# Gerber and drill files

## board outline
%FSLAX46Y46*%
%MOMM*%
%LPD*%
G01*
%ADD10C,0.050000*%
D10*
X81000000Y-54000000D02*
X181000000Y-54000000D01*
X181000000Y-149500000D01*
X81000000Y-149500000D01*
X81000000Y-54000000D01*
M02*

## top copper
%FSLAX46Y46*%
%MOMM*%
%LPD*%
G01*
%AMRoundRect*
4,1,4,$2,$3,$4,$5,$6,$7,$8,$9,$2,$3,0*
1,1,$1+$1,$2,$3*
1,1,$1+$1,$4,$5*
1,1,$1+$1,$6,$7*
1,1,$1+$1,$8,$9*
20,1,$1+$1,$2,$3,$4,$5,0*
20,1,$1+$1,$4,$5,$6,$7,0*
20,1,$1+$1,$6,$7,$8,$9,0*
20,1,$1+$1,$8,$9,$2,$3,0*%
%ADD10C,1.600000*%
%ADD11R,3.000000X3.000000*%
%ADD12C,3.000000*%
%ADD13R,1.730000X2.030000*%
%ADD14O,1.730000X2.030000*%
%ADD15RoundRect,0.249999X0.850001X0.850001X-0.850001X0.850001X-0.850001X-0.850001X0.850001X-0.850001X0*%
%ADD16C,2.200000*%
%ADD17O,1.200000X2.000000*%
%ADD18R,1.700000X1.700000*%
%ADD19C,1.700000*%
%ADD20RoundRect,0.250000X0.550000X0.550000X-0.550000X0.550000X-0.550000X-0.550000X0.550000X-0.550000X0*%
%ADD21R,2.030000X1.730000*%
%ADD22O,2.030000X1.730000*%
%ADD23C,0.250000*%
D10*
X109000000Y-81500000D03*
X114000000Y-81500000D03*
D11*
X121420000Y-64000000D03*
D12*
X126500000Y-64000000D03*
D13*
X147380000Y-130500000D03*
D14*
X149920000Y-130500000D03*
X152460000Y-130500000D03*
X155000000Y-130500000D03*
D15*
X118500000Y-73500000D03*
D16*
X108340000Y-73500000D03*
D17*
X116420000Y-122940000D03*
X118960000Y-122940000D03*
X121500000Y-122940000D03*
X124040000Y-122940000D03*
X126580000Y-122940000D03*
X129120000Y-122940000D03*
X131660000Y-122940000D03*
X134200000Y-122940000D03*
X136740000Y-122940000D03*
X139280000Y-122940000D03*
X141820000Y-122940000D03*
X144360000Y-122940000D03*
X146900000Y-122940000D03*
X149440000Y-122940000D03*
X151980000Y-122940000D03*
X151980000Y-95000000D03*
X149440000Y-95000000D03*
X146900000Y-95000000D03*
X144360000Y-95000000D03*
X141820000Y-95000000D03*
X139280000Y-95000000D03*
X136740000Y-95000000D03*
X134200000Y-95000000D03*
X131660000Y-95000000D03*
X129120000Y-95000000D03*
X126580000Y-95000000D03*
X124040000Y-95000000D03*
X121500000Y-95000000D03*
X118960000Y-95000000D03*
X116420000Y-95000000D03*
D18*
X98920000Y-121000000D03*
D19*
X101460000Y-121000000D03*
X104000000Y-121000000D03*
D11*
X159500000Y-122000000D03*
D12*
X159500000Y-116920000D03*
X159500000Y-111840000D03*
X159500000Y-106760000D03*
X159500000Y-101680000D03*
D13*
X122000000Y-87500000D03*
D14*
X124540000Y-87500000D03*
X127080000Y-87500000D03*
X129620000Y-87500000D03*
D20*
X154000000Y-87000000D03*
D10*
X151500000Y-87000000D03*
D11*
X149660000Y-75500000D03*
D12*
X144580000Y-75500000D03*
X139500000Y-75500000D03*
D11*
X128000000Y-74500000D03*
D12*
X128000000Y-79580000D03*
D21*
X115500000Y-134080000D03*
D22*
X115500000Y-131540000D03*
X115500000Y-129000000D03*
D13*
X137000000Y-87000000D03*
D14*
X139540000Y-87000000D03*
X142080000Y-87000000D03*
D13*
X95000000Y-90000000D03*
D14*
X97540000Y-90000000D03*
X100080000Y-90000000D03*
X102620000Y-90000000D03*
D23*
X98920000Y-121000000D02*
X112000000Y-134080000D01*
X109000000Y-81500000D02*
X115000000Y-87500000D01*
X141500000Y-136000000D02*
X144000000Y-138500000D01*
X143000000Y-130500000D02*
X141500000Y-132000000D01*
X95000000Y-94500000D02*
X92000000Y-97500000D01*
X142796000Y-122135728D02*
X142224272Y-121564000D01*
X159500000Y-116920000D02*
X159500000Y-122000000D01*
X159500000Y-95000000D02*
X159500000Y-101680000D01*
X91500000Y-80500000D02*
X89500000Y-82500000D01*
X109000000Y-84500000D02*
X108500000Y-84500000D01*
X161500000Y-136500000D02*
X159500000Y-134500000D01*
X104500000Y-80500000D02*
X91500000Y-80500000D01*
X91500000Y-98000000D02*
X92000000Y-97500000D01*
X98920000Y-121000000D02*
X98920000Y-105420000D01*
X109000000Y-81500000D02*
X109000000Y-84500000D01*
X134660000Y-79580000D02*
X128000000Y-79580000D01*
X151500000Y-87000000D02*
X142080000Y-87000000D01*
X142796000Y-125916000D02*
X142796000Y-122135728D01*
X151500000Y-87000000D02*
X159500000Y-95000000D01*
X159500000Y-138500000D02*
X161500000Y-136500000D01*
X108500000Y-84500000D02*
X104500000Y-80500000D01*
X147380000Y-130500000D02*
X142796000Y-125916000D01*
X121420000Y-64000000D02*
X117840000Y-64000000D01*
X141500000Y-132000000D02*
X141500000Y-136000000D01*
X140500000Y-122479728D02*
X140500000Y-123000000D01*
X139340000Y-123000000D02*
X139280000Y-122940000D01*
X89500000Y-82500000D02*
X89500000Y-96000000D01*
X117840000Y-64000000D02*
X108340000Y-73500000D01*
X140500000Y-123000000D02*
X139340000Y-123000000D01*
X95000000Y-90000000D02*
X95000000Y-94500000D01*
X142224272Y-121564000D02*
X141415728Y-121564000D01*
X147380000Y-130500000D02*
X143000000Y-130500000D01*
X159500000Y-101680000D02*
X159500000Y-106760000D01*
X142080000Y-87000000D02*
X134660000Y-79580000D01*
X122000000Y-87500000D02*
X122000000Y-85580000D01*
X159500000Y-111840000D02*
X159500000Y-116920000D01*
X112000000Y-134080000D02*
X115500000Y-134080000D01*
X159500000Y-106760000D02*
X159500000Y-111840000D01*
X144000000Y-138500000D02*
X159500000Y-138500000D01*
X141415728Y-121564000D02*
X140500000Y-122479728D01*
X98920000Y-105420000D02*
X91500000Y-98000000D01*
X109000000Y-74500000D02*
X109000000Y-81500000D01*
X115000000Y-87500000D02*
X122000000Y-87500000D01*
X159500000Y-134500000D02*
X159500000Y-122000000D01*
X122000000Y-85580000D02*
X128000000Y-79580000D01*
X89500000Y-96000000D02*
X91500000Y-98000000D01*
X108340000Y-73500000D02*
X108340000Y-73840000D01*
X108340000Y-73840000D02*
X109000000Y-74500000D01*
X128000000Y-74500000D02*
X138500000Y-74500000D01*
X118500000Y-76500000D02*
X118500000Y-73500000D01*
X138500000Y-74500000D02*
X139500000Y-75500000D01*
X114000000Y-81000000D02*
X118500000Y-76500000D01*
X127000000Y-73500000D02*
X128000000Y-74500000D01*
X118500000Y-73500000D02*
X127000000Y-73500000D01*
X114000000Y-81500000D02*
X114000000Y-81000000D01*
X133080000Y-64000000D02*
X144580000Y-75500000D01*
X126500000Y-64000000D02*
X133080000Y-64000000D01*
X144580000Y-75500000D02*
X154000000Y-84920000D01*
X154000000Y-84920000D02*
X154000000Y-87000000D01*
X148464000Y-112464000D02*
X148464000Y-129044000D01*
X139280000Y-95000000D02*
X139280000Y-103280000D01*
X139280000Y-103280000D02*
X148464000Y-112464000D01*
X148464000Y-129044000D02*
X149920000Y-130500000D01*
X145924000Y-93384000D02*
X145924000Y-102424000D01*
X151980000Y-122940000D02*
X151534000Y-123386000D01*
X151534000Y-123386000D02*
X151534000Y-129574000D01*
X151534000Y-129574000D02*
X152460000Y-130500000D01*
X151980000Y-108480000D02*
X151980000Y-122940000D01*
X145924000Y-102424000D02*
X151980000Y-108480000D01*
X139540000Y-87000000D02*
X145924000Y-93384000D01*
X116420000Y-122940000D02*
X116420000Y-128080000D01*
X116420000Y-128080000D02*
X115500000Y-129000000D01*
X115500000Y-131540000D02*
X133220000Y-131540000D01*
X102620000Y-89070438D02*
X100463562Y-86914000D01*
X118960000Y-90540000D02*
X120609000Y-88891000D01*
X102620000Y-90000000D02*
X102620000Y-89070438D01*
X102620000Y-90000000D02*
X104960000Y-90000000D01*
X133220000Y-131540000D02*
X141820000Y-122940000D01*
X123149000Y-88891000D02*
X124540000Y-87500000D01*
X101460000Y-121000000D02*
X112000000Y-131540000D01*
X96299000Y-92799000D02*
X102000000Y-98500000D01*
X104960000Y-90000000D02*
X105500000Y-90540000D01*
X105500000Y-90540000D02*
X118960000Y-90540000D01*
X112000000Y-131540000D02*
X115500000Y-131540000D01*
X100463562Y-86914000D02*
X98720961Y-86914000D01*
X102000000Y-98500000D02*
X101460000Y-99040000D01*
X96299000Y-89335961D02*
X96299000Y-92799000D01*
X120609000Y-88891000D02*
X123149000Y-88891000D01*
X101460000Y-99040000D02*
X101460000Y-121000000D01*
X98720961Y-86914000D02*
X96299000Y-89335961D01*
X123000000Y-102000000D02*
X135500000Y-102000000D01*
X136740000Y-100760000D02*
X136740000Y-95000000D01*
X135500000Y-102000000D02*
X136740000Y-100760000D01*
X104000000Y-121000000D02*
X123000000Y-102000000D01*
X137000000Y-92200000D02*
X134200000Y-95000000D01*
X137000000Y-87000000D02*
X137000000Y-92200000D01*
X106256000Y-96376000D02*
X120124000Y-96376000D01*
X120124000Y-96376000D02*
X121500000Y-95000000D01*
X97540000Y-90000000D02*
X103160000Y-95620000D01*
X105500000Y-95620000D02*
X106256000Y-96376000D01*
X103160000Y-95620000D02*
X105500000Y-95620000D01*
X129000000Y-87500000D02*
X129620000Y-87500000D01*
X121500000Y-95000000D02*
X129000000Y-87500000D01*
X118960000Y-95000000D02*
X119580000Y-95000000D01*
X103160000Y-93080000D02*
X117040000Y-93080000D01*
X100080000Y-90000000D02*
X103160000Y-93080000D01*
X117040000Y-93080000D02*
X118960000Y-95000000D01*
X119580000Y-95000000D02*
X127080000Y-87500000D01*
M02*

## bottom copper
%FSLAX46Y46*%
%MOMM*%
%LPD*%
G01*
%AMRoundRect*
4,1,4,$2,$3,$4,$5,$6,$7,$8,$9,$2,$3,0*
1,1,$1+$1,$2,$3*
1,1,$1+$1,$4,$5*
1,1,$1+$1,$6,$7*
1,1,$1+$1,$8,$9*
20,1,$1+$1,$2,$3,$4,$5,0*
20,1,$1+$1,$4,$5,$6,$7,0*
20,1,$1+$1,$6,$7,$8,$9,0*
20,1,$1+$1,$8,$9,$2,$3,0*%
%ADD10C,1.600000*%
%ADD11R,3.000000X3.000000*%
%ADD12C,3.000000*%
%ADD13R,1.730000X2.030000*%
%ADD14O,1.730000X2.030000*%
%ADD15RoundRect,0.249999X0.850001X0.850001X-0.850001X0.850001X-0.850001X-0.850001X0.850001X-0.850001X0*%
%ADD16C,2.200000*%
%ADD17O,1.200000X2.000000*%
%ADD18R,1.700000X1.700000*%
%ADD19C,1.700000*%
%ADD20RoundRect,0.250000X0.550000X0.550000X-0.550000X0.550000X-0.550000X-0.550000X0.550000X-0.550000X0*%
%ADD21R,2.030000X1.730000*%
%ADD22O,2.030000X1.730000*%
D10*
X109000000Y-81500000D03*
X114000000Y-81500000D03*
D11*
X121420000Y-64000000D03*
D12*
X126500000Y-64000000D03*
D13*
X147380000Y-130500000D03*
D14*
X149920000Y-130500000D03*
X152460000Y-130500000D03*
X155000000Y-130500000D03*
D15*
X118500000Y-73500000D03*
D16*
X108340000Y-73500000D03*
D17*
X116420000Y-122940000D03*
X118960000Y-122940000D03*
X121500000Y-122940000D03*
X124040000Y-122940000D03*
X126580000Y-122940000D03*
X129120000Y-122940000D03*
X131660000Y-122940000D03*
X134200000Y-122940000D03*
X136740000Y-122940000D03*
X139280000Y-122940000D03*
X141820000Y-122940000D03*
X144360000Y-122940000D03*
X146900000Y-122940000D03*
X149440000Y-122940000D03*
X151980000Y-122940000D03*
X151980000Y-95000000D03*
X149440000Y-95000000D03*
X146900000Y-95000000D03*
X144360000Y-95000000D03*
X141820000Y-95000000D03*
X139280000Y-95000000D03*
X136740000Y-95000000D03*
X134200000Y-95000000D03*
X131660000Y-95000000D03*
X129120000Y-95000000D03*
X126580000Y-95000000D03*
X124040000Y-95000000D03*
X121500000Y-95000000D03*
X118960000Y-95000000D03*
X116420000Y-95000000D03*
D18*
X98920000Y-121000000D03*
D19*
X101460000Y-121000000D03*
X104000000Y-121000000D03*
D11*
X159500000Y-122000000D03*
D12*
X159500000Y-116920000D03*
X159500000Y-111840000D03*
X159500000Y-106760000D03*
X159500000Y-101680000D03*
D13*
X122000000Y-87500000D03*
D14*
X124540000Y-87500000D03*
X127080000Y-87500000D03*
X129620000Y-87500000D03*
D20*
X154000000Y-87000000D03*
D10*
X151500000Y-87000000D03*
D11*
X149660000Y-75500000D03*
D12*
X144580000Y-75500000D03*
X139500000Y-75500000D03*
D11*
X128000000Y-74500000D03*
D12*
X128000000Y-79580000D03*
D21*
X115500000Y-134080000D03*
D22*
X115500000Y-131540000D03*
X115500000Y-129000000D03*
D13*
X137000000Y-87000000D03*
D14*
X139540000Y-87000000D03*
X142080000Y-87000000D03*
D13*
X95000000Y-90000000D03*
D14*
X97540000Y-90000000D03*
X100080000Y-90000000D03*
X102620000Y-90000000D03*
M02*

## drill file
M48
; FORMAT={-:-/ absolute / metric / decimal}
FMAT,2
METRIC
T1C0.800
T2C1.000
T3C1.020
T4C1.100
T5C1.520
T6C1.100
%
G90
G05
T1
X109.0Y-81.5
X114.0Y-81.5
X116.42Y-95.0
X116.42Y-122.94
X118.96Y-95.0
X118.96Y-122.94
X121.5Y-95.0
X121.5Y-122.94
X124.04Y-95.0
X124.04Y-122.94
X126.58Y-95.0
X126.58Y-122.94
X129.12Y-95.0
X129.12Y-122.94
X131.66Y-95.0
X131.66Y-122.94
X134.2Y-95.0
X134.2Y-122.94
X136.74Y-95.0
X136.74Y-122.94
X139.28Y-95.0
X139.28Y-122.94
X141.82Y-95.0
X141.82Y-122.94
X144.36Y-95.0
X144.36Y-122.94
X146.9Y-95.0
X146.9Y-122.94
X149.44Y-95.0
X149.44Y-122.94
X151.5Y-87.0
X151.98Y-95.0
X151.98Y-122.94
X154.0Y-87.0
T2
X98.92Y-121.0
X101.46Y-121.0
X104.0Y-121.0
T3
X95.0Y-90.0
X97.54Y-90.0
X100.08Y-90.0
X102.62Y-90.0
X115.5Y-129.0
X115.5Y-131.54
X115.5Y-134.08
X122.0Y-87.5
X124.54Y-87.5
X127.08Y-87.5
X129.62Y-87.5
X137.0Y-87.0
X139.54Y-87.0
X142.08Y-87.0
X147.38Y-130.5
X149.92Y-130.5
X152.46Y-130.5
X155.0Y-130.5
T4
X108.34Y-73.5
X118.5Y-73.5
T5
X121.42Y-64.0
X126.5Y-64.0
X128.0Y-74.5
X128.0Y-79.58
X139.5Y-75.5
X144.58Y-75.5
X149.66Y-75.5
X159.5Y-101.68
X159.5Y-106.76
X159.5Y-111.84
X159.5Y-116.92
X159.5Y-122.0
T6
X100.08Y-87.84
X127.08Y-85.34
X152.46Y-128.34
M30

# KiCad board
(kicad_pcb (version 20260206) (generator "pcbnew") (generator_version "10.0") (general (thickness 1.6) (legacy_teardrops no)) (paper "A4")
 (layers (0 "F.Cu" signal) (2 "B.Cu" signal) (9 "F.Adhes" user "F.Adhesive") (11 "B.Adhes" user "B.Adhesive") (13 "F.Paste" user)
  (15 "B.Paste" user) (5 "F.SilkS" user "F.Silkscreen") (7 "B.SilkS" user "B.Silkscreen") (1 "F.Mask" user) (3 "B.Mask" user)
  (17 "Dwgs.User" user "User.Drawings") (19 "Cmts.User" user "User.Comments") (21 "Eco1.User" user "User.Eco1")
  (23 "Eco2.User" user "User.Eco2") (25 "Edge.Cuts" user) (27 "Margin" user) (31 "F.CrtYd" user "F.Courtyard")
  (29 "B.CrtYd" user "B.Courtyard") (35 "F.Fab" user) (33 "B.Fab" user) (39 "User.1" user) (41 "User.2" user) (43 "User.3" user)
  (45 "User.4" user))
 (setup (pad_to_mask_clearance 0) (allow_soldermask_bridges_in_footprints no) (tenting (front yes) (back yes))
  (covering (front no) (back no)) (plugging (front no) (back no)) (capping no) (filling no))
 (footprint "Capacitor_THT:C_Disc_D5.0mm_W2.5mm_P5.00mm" (layer "F.Cu") (at 109 81.5)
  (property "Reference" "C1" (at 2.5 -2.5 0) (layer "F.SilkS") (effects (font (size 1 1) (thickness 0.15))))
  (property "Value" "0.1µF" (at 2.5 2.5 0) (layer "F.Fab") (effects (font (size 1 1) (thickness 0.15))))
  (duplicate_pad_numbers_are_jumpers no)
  (pad "1" thru_hole circle (at 0 0) (size 1.6 1.6) (drill 0.8) (layers "*.Cu" "*.Mask") (remove_unused_layers no) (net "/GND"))
  (pad "2" thru_hole circle (at 5 0) (size 1.6 1.6) (drill 0.8) (layers "*.Cu" "*.Mask") (remove_unused_layers no) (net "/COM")))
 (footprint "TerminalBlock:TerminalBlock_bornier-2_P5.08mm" (layer "F.Cu") (at 121.42 64)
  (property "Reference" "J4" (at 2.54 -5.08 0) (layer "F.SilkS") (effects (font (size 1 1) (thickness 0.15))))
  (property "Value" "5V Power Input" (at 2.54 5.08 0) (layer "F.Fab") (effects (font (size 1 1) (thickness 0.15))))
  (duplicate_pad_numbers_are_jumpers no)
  (pad "1" thru_hole rect (at 0 0) (size 3 3) (drill 1.52) (layers "*.Cu" "*.Mask") (remove_unused_layers no) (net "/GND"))
  (pad "2" thru_hole circle (at 5.08 0) (size 3 3) (drill 1.52) (layers "*.Cu" "*.Mask") (remove_unused_layers no) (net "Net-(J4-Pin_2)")))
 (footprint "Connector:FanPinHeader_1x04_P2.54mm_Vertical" (layer "F.Cu") (at 147.38 130.5)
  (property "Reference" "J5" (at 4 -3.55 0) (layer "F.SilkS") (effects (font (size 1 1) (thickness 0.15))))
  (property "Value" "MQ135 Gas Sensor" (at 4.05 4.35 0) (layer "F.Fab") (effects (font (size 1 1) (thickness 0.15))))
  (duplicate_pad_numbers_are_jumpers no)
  (pad "" np_thru_hole circle (at 5.08 -2.16 90) (size 1.1 1.1) (drill 1.1) (layers "*.Cu" "*.Mask"))
  (pad "1" thru_hole rect (at 0 0 90) (size 2.03 1.73) (drill 1.02) (layers "*.Cu" "*.Mask") (remove_unused_layers no) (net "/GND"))
  (pad "2" thru_hole oval (at 2.54 0 90) (size 2.03 1.73) (drill 1.02) (layers "*.Cu" "*.Mask") (remove_unused_layers no)
   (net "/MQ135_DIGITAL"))
  (pad "3" thru_hole oval (at 5.08 0 90) (size 2.03 1.73) (drill 1.02) (layers "*.Cu" "*.Mask") (remove_unused_layers no) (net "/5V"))
  (pad "4" thru_hole oval (at 7.62 0 90) (size 2.03 1.73) (drill 1.02) (layers "*.Cu" "*.Mask") (remove_unused_layers no) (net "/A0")))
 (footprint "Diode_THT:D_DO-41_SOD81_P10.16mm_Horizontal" (layer "F.Cu") (at 118.5 73.5 180)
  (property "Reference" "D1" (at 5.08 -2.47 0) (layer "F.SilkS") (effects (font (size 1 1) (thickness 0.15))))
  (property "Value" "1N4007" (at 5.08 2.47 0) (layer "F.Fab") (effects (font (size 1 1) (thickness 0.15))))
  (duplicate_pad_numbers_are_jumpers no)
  (pad "1" thru_hole roundrect (at 0 0 180) (size 2.2 2.2) (drill 1.1) (layers "*.Cu" "*.Mask") (remove_unused_layers no)
   (roundrect_rratio 0.113636) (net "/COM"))
  (pad "2" thru_hole circle (at 10.16 0 180) (size 2.2 2.2) (drill 1.1) (layers "*.Cu" "*.Mask") (remove_unused_layers no) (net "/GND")))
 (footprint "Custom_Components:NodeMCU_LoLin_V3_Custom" (layer "F.Cu") (at 134.2 108.97)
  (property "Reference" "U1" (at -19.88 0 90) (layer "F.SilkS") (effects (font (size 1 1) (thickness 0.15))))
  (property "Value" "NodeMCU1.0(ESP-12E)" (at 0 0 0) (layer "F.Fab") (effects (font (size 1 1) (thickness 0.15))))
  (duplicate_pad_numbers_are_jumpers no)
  (pad "1" thru_hole oval (at -17.78 13.97) (size 1.2 2) (drill 0.8) (layers "*.Cu" "*.Mask") (remove_unused_layers no)
   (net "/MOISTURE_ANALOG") (thermal_bridge_angle 45))
  (pad "2" thru_hole oval (at -15.24 13.97) (size 1.2 2) (drill 0.8) (layers "*.Cu" "*.Mask") (remove_unused_layers no)
   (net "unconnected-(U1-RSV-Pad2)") (thermal_bridge_angle 45))
  (pad "3" thru_hole oval (at -12.7 13.97) (size 1.2 2) (drill 0.8) (layers "*.Cu" "*.Mask") (remove_unused_layers no)
   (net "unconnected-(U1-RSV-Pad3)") (thermal_bridge_angle 45))
  (pad "4" thru_hole oval (at -10.16 13.97) (size 1.2 2) (drill 0.8) (layers "*.Cu" "*.Mask") (remove_unused_layers no)
   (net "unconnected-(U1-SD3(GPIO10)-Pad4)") (thermal_bridge_angle 45))
  (pad "5" thru_hole oval (at -7.62 13.97) (size 1.2 2) (drill 0.8) (layers "*.Cu" "*.Mask") (remove_unused_layers no)
   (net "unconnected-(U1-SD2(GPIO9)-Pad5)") (thermal_bridge_angle 45))
  (pad "6" thru_hole oval (at -5.08 13.97) (size 1.2 2) (drill 0.8) (layers "*.Cu" "*.Mask") (remove_unused_layers no)
   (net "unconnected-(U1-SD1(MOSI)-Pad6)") (thermal_bridge_angle 45))
  (pad "7" thru_hole oval (at -2.54 13.97) (size 1.2 2) (drill 0.8) (layers "*.Cu" "*.Mask") (remove_unused_layers no)
   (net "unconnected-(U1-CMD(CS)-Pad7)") (thermal_bridge_angle 45))
  (pad "8" thru_hole oval (at 0 13.97) (size 1.2 2) (drill 0.8) (layers "*.Cu" "*.Mask") (remove_unused_layers no)
   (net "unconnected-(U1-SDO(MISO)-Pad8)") (thermal_bridge_angle 45))
  (pad "9" thru_hole oval (at 2.54 13.97) (size 1.2 2) (drill 0.8) (layers "*.Cu" "*.Mask") (remove_unused_layers no)
   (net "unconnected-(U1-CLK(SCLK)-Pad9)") (thermal_bridge_angle 45))
  (pad "10" thru_hole oval (at 5.08 13.97) (size 1.2 2) (drill 0.8) (layers "*.Cu" "*.Mask") (remove_unused_layers no) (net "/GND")
   (thermal_bridge_angle 45))
  (pad "11" thru_hole oval (at 7.62 13.97) (size 1.2 2) (drill 0.8) (layers "*.Cu" "*.Mask") (remove_unused_layers no) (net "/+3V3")
   (thermal_bridge_angle 45))
  (pad "12" thru_hole oval (at 10.16 13.97) (size 1.2 2) (drill 0.8) (layers "*.Cu" "*.Mask") (remove_unused_layers no)
   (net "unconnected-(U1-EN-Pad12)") (thermal_bridge_angle 45))
  (pad "13" thru_hole oval (at 12.7 13.97) (size 1.2 2) (drill 0.8) (layers "*.Cu" "*.Mask") (remove_unused_layers no)
   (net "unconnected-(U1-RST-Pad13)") (thermal_bridge_angle 45))
  (pad "14" thru_hole oval (at 15.24 13.97) (size 1.2 2) (drill 0.8) (layers "*.Cu" "*.Mask") (remove_unused_layers no)
   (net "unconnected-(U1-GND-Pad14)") (thermal_bridge_angle 45))
  (pad "15" thru_hole oval (at 17.78 13.97) (size 1.2 2) (drill 0.8) (layers "*.Cu" "*.Mask") (remove_unused_layers no) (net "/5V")
   (thermal_bridge_angle 45))
  (pad "16" thru_hole oval (at 17.78 -13.97) (size 1.2 2) (drill 0.8) (layers "*.Cu" "*.Mask") (remove_unused_layers no)
   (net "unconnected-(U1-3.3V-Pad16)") (thermal_bridge_angle 45))
  (pad "17" thru_hole oval (at 15.24 -13.97) (size 1.2 2) (drill 0.8) (layers "*.Cu" "*.Mask") (remove_unused_layers no)
   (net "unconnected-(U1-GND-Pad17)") (thermal_bridge_angle 45))
  (pad "18" thru_hole oval (at 12.7 -13.97) (size 1.2 2) (drill 0.8) (layers "*.Cu" "*.Mask") (remove_unused_layers no)
   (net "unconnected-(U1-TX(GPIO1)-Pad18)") (thermal_bridge_angle 45))
  (pad "19" thru_hole oval (at 10.16 -13.97) (size 1.2 2) (drill 0.8) (layers "*.Cu" "*.Mask") (remove_unused_layers no)
   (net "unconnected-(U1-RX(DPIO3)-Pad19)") (thermal_bridge_angle 45))
  (pad "20" thru_hole oval (at 7.62 -13.97) (size 1.2 2) (drill 0.8) (layers "*.Cu" "*.Mask") (remove_unused_layers no)
   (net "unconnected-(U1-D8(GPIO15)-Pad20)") (thermal_bridge_angle 45))
  (pad "21" thru_hole oval (at 5.08 -13.97) (size 1.2 2) (drill 0.8) (layers "*.Cu" "*.Mask") (remove_unused_layers no)
   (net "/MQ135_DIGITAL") (thermal_bridge_angle 45))
  (pad "22" thru_hole oval (at 2.54 -13.97) (size 1.2 2) (drill 0.8) (layers "*.Cu" "*.Mask") (remove_unused_layers no) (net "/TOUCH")
   (thermal_bridge_angle 45))
  (pad "23" thru_hole oval (at 0 -13.97) (size 1.2 2) (drill 0.8) (layers "*.Cu" "*.Mask") (remove_unused_layers no) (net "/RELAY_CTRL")
   (thermal_bridge_angle 45))
  (pad "24" thru_hole oval (at -2.54 -13.97) (size 1.2 2) (drill 0.8) (layers "*.Cu" "*.Mask") (remove_unused_layers no)
   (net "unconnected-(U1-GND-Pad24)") (thermal_bridge_angle 45))
  (pad "25" thru_hole oval (at -5.08 -13.97) (size 1.2 2) (drill 0.8) (layers "*.Cu" "*.Mask") (remove_unused_layers no)
   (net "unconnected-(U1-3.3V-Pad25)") (thermal_bridge_angle 45))
  (pad "26" thru_hole oval (at -7.62 -13.97) (size 1.2 2) (drill 0.8) (layers "*.Cu" "*.Mask") (remove_unused_layers no)
   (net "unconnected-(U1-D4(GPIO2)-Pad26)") (thermal_bridge_angle 45))
  (pad "27" thru_hole oval (at -10.16 -13.97) (size 1.2 2) (drill 0.8) (layers "*.Cu" "*.Mask") (remove_unused_layers no)
   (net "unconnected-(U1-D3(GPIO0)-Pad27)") (thermal_bridge_angle 45))
  (pad "28" thru_hole oval (at -12.7 -13.97) (size 1.2 2) (drill 0.8) (layers "*.Cu" "*.Mask") (remove_unused_layers no) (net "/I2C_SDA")
   (thermal_bridge_angle 45))
  (pad "29" thru_hole oval (at -15.24 -13.97) (size 1.2 2) (drill 0.8) (layers "*.Cu" "*.Mask") (remove_unused_layers no) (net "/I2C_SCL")
   (thermal_bridge_angle 45))
  (pad "30" thru_hole oval (at -17.78 -13.97) (size 1.2 2) (drill 0.8) (layers "*.Cu" "*.Mask") (remove_unused_layers no)
   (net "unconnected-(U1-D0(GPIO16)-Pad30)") (thermal_bridge_angle 45)))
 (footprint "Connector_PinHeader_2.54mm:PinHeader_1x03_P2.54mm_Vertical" (layer "F.Cu") (at 98.92 121 90)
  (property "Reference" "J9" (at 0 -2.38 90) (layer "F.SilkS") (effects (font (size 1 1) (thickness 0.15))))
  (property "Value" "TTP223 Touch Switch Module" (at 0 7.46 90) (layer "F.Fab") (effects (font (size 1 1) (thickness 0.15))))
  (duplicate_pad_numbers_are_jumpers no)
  (pad "1" thru_hole rect (at 0 0 90) (size 1.7 1.7) (drill 1) (layers "*.Cu" "*.Mask") (remove_unused_layers no) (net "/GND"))
  (pad "2" thru_hole circle (at 0 2.54 90) (size 1.7 1.7) (drill 1) (layers "*.Cu" "*.Mask") (remove_unused_layers no) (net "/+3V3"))
  (pad "3" thru_hole circle (at 0 5.08 90) (size 1.7 1.7) (drill 1) (layers "*.Cu" "*.Mask") (remove_unused_layers no) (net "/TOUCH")))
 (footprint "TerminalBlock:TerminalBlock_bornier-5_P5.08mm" (layer "F.Cu") (at 159.5 122 90)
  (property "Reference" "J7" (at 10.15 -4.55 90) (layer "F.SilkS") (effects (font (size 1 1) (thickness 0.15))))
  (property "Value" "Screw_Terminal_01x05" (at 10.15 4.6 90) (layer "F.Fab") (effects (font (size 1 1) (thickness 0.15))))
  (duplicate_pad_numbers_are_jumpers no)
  (pad "1" thru_hole rect (at 0 0 90) (size 3 3) (drill 1.52) (layers "*.Cu" "*.Mask") (remove_unused_layers no) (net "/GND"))
  (pad "2" thru_hole circle (at 5.08 0 90) (size 3 3) (drill 1.52) (layers "*.Cu" "*.Mask") (remove_unused_layers no) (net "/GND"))
  (pad "3" thru_hole circle (at 10.16 0 90) (size 3 3) (drill 1.52) (layers "*.Cu" "*.Mask") (remove_unused_layers no) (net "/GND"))
  (pad "4" thru_hole circle (at 15.24 0 90) (size 3 3) (drill 1.52) (layers "*.Cu" "*.Mask") (remove_unused_layers no) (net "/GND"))
  (pad "5" thru_hole circle (at 20.32 0 90) (size 3 3) (drill 1.52) (layers "*.Cu" "*.Mask") (remove_unused_layers no) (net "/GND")))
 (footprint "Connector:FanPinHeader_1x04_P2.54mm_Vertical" (layer "F.Cu") (at 122 87.5)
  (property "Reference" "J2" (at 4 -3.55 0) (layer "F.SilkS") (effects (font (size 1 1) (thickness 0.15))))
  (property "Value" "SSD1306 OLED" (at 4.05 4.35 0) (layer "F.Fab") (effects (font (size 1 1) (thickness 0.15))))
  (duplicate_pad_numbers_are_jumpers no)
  (pad "" np_thru_hole circle (at 5.08 -2.16 90) (size 1.1 1.1) (drill 1.1) (layers "*.Cu" "*.Mask"))
  (pad "1" thru_hole rect (at 0 0 90) (size 2.03 1.73) (drill 1.02) (layers "*.Cu" "*.Mask") (remove_unused_layers no) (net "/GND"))
  (pad "2" thru_hole oval (at 2.54 0 90) (size 2.03 1.73) (drill 1.02) (layers "*.Cu" "*.Mask") (remove_unused_layers no) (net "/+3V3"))
  (pad "3" thru_hole oval (at 5.08 0 90) (size 2.03 1.73) (drill 1.02) (layers "*.Cu" "*.Mask") (remove_unused_layers no) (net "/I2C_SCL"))
  (pad "4" thru_hole oval (at 7.62 0 90) (size 2.03 1.73) (drill 1.02) (layers "*.Cu" "*.Mask") (remove_unused_layers no) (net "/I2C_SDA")))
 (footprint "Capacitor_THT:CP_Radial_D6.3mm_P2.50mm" (layer "F.Cu") (at 154 87 180)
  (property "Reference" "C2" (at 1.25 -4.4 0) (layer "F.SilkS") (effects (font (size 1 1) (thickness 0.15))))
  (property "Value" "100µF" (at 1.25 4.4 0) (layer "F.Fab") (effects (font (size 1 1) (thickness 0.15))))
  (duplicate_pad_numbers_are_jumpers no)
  (pad "1" thru_hole roundrect (at 0 0 180) (size 1.6 1.6) (drill 0.8) (layers "*.Cu" "*.Mask") (remove_unused_layers no)
   (roundrect_rratio 0.15625) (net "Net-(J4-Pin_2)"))
  (pad "2" thru_hole circle (at 2.5 0 180) (size 1.6 1.6) (drill 0.8) (layers "*.Cu" "*.Mask") (remove_unused_layers no) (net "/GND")))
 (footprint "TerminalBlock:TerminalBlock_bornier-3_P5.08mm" (layer "F.Cu") (at 149.66 75.5 180)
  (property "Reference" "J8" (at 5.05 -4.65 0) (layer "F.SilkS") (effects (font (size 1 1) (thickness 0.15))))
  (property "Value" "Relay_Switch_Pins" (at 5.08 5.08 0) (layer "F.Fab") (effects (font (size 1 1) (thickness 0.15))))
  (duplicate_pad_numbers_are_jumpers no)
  (pad "1" thru_hole rect (at 0 0 180) (size 3 3) (drill 1.52) (layers "*.Cu" "*.Mask") (remove_unused_layers no)
   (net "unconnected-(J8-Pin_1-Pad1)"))
  (pad "2" thru_hole circle (at 5.08 0 180) (size 3 3) (drill 1.52) (layers "*.Cu" "*.Mask") (remove_unused_layers no)
   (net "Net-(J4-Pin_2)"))
  (pad "3" thru_hole circle (at 10.16 0 180) (size 3 3) (drill 1.52) (layers "*.Cu" "*.Mask") (remove_unused_layers no) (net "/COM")))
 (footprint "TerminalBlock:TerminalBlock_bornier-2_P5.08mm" (layer "F.Cu") (at 128 74.5 -90)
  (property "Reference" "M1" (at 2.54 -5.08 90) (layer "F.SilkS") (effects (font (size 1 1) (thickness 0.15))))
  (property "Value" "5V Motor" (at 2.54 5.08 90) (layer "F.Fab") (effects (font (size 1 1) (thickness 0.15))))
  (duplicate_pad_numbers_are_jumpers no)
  (pad "1" thru_hole rect (at 0 0 270) (size 3 3) (drill 1.52) (layers "*.Cu" "*.Mask") (remove_unused_layers no) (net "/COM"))
  (pad "2" thru_hole circle (at 5.08 0 270) (size 3 3) (drill 1.52) (layers "*.Cu" "*.Mask") (remove_unused_layers no) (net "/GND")))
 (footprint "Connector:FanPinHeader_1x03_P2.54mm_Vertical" (layer "F.Cu") (at 115.5 134.08 90)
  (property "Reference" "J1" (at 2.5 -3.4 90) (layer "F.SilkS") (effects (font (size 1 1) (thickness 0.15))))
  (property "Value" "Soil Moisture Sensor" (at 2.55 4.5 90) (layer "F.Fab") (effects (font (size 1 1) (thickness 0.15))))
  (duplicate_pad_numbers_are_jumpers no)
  (pad "1" thru_hole rect (at 0 0 180) (size 2.03 1.73) (drill 1.02) (layers "*.Cu" "*.Mask") (remove_unused_layers no) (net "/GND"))
  (pad "2" thru_hole oval (at 2.54 0 180) (size 2.03 1.73) (drill 1.02) (layers "*.Cu" "*.Mask") (remove_unused_layers no) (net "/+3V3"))
  (pad "3" thru_hole oval (at 5.08 0 180) (size 2.03 1.73) (drill 1.02) (layers "*.Cu" "*.Mask") (remove_unused_layers no)
   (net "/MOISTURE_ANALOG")))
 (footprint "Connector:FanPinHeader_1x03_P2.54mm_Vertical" (layer "F.Cu") (at 137 87)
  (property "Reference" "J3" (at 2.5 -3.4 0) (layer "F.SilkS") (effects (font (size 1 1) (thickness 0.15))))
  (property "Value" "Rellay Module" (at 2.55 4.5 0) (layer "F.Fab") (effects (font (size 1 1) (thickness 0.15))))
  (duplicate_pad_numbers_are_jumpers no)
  (pad "1" thru_hole rect (at 0 0 90) (size 2.03 1.73) (drill 1.02) (layers "*.Cu" "*.Mask") (remove_unused_layers no) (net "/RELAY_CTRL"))
  (pad "2" thru_hole oval (at 2.54 0 90) (size 2.03 1.73) (drill 1.02) (layers "*.Cu" "*.Mask") (remove_unused_layers no) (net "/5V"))
  (pad "3" thru_hole oval (at 5.08 0 90) (size 2.03 1.73) (drill 1.02) (layers "*.Cu" "*.Mask") (remove_unused_layers no) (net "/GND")))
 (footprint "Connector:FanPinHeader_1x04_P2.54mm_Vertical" (layer "F.Cu") (at 95 90)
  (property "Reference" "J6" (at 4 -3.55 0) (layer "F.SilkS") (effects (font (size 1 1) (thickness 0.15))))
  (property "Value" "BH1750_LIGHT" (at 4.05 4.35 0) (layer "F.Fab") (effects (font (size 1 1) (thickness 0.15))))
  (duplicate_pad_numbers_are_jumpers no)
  (pad "" np_thru_hole circle (at 5.08 -2.16 90) (size 1.1 1.1) (drill 1.1) (layers "*.Cu" "*.Mask"))
  (pad "1" thru_hole rect (at 0 0 90) (size 2.03 1.73) (drill 1.02) (layers "*.Cu" "*.Mask") (remove_unused_layers no) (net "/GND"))
  (pad "2" thru_hole oval (at 2.54 0 90) (size 2.03 1.73) (drill 1.02) (layers "*.Cu" "*.Mask") (remove_unused_layers no) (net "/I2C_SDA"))
  (pad "3" thru_hole oval (at 5.08 0 90) (size 2.03 1.73) (drill 1.02) (layers "*.Cu" "*.Mask") (remove_unused_layers no) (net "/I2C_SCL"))
  (pad "4" thru_hole oval (at 7.62 0 90) (size 2.03 1.73) (drill 1.02) (layers "*.Cu" "*.Mask") (remove_unused_layers no) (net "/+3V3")))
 (gr_rect (start 81 54) (end 181 149.5) (stroke (width 0.05) (type default)) (fill no) (layer "Edge.Cuts"))
 (segment (start 98.92 121) (end 112 134.08) (width 0.25) (layer "F.Cu") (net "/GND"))
 (segment (start 109 81.5) (end 115 87.5) (width 0.25) (layer "F.Cu") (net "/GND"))
 (segment (start 141.5 136) (end 144 138.5) (width 0.25) (layer "F.Cu") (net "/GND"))
 (segment (start 143 130.5) (end 141.5 132) (width 0.25) (layer "F.Cu") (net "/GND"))
 (segment (start 95 94.5) (end 92 97.5) (width 0.25) (layer "F.Cu") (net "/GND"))
 (segment (start 142.796 122.135728) (end 142.224272 121.564) (width 0.25) (layer "F.Cu") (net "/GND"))
 (segment (start 159.5 116.92) (end 159.5 122) (width 0.25) (layer "F.Cu") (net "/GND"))
 (segment (start 159.5 95) (end 159.5 101.68) (width 0.25) (layer "F.Cu") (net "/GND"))
 (segment (start 91.5 80.5) (end 89.5 82.5) (width 0.25) (layer "F.Cu") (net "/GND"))
 (segment (start 109 84.5) (end 108.5 84.5) (width 0.25) (layer "F.Cu") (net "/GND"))
 (segment (start 161.5 136.5) (end 159.5 134.5) (width 0.25) (layer "F.Cu") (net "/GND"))
 (segment (start 104.5 80.5) (end 91.5 80.5) (width 0.25) (layer "F.Cu") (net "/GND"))
 (segment (start 91.5 98) (end 92 97.5) (width 0.25) (layer "F.Cu") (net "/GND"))
 (segment (start 98.92 121) (end 98.92 105.42) (width 0.25) (layer "F.Cu") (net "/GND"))
 (segment (start 109 81.5) (end 109 84.5) (width 0.25) (layer "F.Cu") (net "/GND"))
 (segment (start 134.66 79.58) (end 128 79.58) (width 0.25) (layer "F.Cu") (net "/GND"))
 (segment (start 151.5 87) (end 142.08 87) (width 0.25) (layer "F.Cu") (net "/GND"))
 (segment (start 142.796 125.916) (end 142.796 122.135728) (width 0.25) (layer "F.Cu") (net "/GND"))
 (segment (start 151.5 87) (end 159.5 95) (width 0.25) (layer "F.Cu") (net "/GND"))
 (segment (start 159.5 138.5) (end 161.5 136.5) (width 0.25) (layer "F.Cu") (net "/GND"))
 (segment (start 108.5 84.5) (end 104.5 80.5) (width 0.25) (layer "F.Cu") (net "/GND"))
 (segment (start 147.38 130.5) (end 142.796 125.916) (width 0.25) (layer "F.Cu") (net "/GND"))
 (segment (start 121.42 64) (end 117.84 64) (width 0.25) (layer "F.Cu") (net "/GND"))
 (segment (start 141.5 132) (end 141.5 136) (width 0.25) (layer "F.Cu") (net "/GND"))
 (segment (start 140.5 122.479728) (end 140.5 123) (width 0.25) (layer "F.Cu") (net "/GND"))
 (segment (start 139.34 123) (end 139.28 122.94) (width 0.25) (layer "F.Cu") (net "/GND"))
 (segment (start 89.5 82.5) (end 89.5 96) (width 0.25) (layer "F.Cu") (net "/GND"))
 (segment (start 117.84 64) (end 108.34 73.5) (width 0.25) (layer "F.Cu") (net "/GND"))
 (segment (start 140.5 123) (end 139.34 123) (width 0.25) (layer "F.Cu") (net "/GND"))
 (segment (start 95 90) (end 95 94.5) (width 0.25) (layer "F.Cu") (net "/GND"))
 (segment (start 142.224272 121.564) (end 141.415728 121.564) (width 0.25) (layer "F.Cu") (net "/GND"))
 (segment (start 147.38 130.5) (end 143 130.5) (width 0.25) (layer "F.Cu") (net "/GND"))
 (segment (start 159.5 101.68) (end 159.5 106.76) (width 0.25) (layer "F.Cu") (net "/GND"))
 (segment (start 142.08 87) (end 134.66 79.58) (width 0.25) (layer "F.Cu") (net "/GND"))
 (segment (start 122 87.5) (end 122 85.58) (width 0.25) (layer "F.Cu") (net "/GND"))
 (segment (start 159.5 111.84) (end 159.5 116.92) (width 0.25) (layer "F.Cu") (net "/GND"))
 (segment (start 112 134.08) (end 115.5 134.08) (width 0.25) (layer "F.Cu") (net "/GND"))
 (segment (start 159.5 106.76) (end 159.5 111.84) (width 0.25) (layer "F.Cu") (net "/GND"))
 (segment (start 144 138.5) (end 159.5 138.5) (width 0.25) (layer "F.Cu") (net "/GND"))
 (segment (start 141.415728 121.564) (end 140.5 122.479728) (width 0.25) (layer "F.Cu") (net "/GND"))
 (segment (start 98.92 105.42) (end 91.5 98) (width 0.25) (layer "F.Cu") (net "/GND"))
 (segment (start 109 74.5) (end 109 81.5) (width 0.25) (layer "F.Cu") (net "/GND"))
 (segment (start 115 87.5) (end 122 87.5) (width 0.25) (layer "F.Cu") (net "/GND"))
 (segment (start 159.5 134.5) (end 159.5 122) (width 0.25) (layer "F.Cu") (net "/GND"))
 (segment (start 122 85.58) (end 128 79.58) (width 0.25) (layer "F.Cu") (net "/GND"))
 (segment (start 89.5 96) (end 91.5 98) (width 0.25) (layer "F.Cu") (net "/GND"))
 (segment (start 108.34 73.5) (end 108.34 73.84) (width 0.25) (layer "F.Cu") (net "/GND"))
 (segment (start 108.34 73.84) (end 109 74.5) (width 0.25) (layer "F.Cu") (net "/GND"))
 (segment (start 128 74.5) (end 138.5 74.5) (width 0.25) (layer "F.Cu") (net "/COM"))
 (segment (start 118.5 76.5) (end 118.5 73.5) (width 0.25) (layer "F.Cu") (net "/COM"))
 (segment (start 138.5 74.5) (end 139.5 75.5) (width 0.25) (layer "F.Cu") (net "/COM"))
 (segment (start 114 81) (end 118.5 76.5) (width 0.25) (layer "F.Cu") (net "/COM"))
 (segment (start 127 73.5) (end 128 74.5) (width 0.25) (layer "F.Cu") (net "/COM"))
 (segment (start 118.5 73.5) (end 127 73.5) (width 0.25) (layer "F.Cu") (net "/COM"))
 (segment (start 114 81.5) (end 114 81) (width 0.25) (layer "F.Cu") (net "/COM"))
 (segment (start 133.08 64) (end 144.58 75.5) (width 0.25) (layer "F.Cu") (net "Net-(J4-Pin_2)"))
 (segment (start 126.5 64) (end 133.08 64) (width 0.25) (layer "F.Cu") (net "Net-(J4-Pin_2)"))
 (segment (start 144.58 75.5) (end 154 84.92) (width 0.25) (layer "F.Cu") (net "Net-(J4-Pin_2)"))
 (segment (start 154 84.92) (end 154 87) (width 0.25) (layer "F.Cu") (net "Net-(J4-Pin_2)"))
 (segment (start 148.464 112.464) (end 148.464 129.044) (width 0.25) (layer "F.Cu") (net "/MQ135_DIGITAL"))
 (segment (start 139.28 95) (end 139.28 103.28) (width 0.25) (layer "F.Cu") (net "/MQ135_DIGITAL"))
 (segment (start 139.28 103.28) (end 148.464 112.464) (width 0.25) (layer "F.Cu") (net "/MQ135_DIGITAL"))
 (segment (start 148.464 129.044) (end 149.92 130.5) (width 0.25) (layer "F.Cu") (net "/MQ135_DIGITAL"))
 (segment (start 145.924 93.384) (end 145.924 102.424) (width 0.25) (layer "F.Cu") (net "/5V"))
 (segment (start 151.98 122.94) (end 151.534 123.386) (width 0.25) (layer "F.Cu") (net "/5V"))
 (segment (start 151.534 123.386) (end 151.534 129.574) (width 0.25) (layer "F.Cu") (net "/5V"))
 (segment (start 151.534 129.574) (end 152.46 130.5) (width 0.25) (layer "F.Cu") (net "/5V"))
 (segment (start 151.98 108.48) (end 151.98 122.94) (width 0.25) (layer "F.Cu") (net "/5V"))
 (segment (start 145.924 102.424) (end 151.98 108.48) (width 0.25) (layer "F.Cu") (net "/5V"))
 (segment (start 139.54 87) (end 145.924 93.384) (width 0.25) (layer "F.Cu") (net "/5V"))
 (segment (start 116.42 122.94) (end 116.42 128.08) (width 0.25) (layer "F.Cu") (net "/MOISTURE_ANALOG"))
 (segment (start 116.42 128.08) (end 115.5 129) (width 0.25) (layer "F.Cu") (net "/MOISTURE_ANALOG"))
 (segment (start 115.5 131.54) (end 133.22 131.54) (width 0.25) (layer "F.Cu") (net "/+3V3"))
 (segment (start 102.62 89.070438) (end 100.463562 86.914) (width 0.25) (layer "F.Cu") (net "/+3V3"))
 (segment (start 118.96 90.54) (end 120.609 88.891) (width 0.25) (layer "F.Cu") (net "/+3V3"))
 (segment (start 102.62 90) (end 102.62 89.070438) (width 0.25) (layer "F.Cu") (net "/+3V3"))
 (segment (start 102.62 90) (end 104.96 90) (width 0.25) (layer "F.Cu") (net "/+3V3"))
 (segment (start 133.22 131.54) (end 141.82 122.94) (width 0.25) (layer "F.Cu") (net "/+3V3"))
 (segment (start 123.149 88.891) (end 124.54 87.5) (width 0.25) (layer "F.Cu") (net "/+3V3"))
 (segment (start 101.46 121) (end 112 131.54) (width 0.25) (layer "F.Cu") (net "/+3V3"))
 (segment (start 96.299 92.799) (end 102 98.5) (width 0.25) (layer "F.Cu") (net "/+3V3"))
 (segment (start 104.96 90) (end 105.5 90.54) (width 0.25) (layer "F.Cu") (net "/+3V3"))
 (segment (start 105.5 90.54) (end 118.96 90.54) (width 0.25) (layer "F.Cu") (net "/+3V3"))
 (segment (start 112 131.54) (end 115.5 131.54) (width 0.25) (layer "F.Cu") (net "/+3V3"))
 (segment (start 100.463562 86.914) (end 98.720961 86.914) (width 0.25) (layer "F.Cu") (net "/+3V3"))
 (segment (start 102 98.5) (end 101.46 99.04) (width 0.25) (layer "F.Cu") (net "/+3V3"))
 (segment (start 96.299 89.335961) (end 96.299 92.799) (width 0.25) (layer "F.Cu") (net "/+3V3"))
 (segment (start 120.609 88.891) (end 123.149 88.891) (width 0.25) (layer "F.Cu") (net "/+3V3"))
 (segment (start 101.46 99.04) (end 101.46 121) (width 0.25) (layer "F.Cu") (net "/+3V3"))
 (segment (start 98.720961 86.914) (end 96.299 89.335961) (width 0.25) (layer "F.Cu") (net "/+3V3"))
 (segment (start 123 102) (end 135.5 102) (width 0.25) (layer "F.Cu") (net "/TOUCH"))
 (segment (start 136.74 100.76) (end 136.74 95) (width 0.25) (layer "F.Cu") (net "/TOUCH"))
 (segment (start 135.5 102) (end 136.74 100.76) (width 0.25) (layer "F.Cu") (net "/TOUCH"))
 (segment (start 104 121) (end 123 102) (width 0.25) (layer "F.Cu") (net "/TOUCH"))
 (segment (start 137 92.2) (end 134.2 95) (width 0.25) (layer "F.Cu") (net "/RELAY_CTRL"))
 (segment (start 137 87) (end 137 92.2) (width 0.25) (layer "F.Cu") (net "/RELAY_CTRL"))
 (segment (start 106.256 96.376) (end 120.124 96.376) (width 0.25) (layer "F.Cu") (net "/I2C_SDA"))
 (segment (start 120.124 96.376) (end 121.5 95) (width 0.25) (layer "F.Cu") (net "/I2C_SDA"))
 (segment (start 97.54 90) (end 103.16 95.62) (width 0.25) (layer "F.Cu") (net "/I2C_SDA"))
 (segment (start 105.5 95.62) (end 106.256 96.376) (width 0.25) (layer "F.Cu") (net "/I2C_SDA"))
 (segment (start 103.16 95.62) (end 105.5 95.62) (width 0.25) (layer "F.Cu") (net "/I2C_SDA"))
 (segment (start 129 87.5) (end 129.62 87.5) (width 0.25) (layer "F.Cu") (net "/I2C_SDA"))
 (segment (start 121.5 95) (end 129 87.5) (width 0.25) (layer "F.Cu") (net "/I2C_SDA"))
 (segment (start 118.96 95) (end 119.58 95) (width 0.25) (layer "F.Cu") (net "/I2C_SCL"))
 (segment (start 103.16 93.08) (end 117.04 93.08) (width 0.25) (layer "F.Cu") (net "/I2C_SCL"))
 (segment (start 100.08 90) (end 103.16 93.08) (width 0.25) (layer "F.Cu") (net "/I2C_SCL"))
 (segment (start 117.04 93.08) (end 118.96 95) (width 0.25) (layer "F.Cu") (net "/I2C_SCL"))
 (segment (start 119.58 95) (end 127.08 87.5) (width 0.25) (layer "F.Cu") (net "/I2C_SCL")))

